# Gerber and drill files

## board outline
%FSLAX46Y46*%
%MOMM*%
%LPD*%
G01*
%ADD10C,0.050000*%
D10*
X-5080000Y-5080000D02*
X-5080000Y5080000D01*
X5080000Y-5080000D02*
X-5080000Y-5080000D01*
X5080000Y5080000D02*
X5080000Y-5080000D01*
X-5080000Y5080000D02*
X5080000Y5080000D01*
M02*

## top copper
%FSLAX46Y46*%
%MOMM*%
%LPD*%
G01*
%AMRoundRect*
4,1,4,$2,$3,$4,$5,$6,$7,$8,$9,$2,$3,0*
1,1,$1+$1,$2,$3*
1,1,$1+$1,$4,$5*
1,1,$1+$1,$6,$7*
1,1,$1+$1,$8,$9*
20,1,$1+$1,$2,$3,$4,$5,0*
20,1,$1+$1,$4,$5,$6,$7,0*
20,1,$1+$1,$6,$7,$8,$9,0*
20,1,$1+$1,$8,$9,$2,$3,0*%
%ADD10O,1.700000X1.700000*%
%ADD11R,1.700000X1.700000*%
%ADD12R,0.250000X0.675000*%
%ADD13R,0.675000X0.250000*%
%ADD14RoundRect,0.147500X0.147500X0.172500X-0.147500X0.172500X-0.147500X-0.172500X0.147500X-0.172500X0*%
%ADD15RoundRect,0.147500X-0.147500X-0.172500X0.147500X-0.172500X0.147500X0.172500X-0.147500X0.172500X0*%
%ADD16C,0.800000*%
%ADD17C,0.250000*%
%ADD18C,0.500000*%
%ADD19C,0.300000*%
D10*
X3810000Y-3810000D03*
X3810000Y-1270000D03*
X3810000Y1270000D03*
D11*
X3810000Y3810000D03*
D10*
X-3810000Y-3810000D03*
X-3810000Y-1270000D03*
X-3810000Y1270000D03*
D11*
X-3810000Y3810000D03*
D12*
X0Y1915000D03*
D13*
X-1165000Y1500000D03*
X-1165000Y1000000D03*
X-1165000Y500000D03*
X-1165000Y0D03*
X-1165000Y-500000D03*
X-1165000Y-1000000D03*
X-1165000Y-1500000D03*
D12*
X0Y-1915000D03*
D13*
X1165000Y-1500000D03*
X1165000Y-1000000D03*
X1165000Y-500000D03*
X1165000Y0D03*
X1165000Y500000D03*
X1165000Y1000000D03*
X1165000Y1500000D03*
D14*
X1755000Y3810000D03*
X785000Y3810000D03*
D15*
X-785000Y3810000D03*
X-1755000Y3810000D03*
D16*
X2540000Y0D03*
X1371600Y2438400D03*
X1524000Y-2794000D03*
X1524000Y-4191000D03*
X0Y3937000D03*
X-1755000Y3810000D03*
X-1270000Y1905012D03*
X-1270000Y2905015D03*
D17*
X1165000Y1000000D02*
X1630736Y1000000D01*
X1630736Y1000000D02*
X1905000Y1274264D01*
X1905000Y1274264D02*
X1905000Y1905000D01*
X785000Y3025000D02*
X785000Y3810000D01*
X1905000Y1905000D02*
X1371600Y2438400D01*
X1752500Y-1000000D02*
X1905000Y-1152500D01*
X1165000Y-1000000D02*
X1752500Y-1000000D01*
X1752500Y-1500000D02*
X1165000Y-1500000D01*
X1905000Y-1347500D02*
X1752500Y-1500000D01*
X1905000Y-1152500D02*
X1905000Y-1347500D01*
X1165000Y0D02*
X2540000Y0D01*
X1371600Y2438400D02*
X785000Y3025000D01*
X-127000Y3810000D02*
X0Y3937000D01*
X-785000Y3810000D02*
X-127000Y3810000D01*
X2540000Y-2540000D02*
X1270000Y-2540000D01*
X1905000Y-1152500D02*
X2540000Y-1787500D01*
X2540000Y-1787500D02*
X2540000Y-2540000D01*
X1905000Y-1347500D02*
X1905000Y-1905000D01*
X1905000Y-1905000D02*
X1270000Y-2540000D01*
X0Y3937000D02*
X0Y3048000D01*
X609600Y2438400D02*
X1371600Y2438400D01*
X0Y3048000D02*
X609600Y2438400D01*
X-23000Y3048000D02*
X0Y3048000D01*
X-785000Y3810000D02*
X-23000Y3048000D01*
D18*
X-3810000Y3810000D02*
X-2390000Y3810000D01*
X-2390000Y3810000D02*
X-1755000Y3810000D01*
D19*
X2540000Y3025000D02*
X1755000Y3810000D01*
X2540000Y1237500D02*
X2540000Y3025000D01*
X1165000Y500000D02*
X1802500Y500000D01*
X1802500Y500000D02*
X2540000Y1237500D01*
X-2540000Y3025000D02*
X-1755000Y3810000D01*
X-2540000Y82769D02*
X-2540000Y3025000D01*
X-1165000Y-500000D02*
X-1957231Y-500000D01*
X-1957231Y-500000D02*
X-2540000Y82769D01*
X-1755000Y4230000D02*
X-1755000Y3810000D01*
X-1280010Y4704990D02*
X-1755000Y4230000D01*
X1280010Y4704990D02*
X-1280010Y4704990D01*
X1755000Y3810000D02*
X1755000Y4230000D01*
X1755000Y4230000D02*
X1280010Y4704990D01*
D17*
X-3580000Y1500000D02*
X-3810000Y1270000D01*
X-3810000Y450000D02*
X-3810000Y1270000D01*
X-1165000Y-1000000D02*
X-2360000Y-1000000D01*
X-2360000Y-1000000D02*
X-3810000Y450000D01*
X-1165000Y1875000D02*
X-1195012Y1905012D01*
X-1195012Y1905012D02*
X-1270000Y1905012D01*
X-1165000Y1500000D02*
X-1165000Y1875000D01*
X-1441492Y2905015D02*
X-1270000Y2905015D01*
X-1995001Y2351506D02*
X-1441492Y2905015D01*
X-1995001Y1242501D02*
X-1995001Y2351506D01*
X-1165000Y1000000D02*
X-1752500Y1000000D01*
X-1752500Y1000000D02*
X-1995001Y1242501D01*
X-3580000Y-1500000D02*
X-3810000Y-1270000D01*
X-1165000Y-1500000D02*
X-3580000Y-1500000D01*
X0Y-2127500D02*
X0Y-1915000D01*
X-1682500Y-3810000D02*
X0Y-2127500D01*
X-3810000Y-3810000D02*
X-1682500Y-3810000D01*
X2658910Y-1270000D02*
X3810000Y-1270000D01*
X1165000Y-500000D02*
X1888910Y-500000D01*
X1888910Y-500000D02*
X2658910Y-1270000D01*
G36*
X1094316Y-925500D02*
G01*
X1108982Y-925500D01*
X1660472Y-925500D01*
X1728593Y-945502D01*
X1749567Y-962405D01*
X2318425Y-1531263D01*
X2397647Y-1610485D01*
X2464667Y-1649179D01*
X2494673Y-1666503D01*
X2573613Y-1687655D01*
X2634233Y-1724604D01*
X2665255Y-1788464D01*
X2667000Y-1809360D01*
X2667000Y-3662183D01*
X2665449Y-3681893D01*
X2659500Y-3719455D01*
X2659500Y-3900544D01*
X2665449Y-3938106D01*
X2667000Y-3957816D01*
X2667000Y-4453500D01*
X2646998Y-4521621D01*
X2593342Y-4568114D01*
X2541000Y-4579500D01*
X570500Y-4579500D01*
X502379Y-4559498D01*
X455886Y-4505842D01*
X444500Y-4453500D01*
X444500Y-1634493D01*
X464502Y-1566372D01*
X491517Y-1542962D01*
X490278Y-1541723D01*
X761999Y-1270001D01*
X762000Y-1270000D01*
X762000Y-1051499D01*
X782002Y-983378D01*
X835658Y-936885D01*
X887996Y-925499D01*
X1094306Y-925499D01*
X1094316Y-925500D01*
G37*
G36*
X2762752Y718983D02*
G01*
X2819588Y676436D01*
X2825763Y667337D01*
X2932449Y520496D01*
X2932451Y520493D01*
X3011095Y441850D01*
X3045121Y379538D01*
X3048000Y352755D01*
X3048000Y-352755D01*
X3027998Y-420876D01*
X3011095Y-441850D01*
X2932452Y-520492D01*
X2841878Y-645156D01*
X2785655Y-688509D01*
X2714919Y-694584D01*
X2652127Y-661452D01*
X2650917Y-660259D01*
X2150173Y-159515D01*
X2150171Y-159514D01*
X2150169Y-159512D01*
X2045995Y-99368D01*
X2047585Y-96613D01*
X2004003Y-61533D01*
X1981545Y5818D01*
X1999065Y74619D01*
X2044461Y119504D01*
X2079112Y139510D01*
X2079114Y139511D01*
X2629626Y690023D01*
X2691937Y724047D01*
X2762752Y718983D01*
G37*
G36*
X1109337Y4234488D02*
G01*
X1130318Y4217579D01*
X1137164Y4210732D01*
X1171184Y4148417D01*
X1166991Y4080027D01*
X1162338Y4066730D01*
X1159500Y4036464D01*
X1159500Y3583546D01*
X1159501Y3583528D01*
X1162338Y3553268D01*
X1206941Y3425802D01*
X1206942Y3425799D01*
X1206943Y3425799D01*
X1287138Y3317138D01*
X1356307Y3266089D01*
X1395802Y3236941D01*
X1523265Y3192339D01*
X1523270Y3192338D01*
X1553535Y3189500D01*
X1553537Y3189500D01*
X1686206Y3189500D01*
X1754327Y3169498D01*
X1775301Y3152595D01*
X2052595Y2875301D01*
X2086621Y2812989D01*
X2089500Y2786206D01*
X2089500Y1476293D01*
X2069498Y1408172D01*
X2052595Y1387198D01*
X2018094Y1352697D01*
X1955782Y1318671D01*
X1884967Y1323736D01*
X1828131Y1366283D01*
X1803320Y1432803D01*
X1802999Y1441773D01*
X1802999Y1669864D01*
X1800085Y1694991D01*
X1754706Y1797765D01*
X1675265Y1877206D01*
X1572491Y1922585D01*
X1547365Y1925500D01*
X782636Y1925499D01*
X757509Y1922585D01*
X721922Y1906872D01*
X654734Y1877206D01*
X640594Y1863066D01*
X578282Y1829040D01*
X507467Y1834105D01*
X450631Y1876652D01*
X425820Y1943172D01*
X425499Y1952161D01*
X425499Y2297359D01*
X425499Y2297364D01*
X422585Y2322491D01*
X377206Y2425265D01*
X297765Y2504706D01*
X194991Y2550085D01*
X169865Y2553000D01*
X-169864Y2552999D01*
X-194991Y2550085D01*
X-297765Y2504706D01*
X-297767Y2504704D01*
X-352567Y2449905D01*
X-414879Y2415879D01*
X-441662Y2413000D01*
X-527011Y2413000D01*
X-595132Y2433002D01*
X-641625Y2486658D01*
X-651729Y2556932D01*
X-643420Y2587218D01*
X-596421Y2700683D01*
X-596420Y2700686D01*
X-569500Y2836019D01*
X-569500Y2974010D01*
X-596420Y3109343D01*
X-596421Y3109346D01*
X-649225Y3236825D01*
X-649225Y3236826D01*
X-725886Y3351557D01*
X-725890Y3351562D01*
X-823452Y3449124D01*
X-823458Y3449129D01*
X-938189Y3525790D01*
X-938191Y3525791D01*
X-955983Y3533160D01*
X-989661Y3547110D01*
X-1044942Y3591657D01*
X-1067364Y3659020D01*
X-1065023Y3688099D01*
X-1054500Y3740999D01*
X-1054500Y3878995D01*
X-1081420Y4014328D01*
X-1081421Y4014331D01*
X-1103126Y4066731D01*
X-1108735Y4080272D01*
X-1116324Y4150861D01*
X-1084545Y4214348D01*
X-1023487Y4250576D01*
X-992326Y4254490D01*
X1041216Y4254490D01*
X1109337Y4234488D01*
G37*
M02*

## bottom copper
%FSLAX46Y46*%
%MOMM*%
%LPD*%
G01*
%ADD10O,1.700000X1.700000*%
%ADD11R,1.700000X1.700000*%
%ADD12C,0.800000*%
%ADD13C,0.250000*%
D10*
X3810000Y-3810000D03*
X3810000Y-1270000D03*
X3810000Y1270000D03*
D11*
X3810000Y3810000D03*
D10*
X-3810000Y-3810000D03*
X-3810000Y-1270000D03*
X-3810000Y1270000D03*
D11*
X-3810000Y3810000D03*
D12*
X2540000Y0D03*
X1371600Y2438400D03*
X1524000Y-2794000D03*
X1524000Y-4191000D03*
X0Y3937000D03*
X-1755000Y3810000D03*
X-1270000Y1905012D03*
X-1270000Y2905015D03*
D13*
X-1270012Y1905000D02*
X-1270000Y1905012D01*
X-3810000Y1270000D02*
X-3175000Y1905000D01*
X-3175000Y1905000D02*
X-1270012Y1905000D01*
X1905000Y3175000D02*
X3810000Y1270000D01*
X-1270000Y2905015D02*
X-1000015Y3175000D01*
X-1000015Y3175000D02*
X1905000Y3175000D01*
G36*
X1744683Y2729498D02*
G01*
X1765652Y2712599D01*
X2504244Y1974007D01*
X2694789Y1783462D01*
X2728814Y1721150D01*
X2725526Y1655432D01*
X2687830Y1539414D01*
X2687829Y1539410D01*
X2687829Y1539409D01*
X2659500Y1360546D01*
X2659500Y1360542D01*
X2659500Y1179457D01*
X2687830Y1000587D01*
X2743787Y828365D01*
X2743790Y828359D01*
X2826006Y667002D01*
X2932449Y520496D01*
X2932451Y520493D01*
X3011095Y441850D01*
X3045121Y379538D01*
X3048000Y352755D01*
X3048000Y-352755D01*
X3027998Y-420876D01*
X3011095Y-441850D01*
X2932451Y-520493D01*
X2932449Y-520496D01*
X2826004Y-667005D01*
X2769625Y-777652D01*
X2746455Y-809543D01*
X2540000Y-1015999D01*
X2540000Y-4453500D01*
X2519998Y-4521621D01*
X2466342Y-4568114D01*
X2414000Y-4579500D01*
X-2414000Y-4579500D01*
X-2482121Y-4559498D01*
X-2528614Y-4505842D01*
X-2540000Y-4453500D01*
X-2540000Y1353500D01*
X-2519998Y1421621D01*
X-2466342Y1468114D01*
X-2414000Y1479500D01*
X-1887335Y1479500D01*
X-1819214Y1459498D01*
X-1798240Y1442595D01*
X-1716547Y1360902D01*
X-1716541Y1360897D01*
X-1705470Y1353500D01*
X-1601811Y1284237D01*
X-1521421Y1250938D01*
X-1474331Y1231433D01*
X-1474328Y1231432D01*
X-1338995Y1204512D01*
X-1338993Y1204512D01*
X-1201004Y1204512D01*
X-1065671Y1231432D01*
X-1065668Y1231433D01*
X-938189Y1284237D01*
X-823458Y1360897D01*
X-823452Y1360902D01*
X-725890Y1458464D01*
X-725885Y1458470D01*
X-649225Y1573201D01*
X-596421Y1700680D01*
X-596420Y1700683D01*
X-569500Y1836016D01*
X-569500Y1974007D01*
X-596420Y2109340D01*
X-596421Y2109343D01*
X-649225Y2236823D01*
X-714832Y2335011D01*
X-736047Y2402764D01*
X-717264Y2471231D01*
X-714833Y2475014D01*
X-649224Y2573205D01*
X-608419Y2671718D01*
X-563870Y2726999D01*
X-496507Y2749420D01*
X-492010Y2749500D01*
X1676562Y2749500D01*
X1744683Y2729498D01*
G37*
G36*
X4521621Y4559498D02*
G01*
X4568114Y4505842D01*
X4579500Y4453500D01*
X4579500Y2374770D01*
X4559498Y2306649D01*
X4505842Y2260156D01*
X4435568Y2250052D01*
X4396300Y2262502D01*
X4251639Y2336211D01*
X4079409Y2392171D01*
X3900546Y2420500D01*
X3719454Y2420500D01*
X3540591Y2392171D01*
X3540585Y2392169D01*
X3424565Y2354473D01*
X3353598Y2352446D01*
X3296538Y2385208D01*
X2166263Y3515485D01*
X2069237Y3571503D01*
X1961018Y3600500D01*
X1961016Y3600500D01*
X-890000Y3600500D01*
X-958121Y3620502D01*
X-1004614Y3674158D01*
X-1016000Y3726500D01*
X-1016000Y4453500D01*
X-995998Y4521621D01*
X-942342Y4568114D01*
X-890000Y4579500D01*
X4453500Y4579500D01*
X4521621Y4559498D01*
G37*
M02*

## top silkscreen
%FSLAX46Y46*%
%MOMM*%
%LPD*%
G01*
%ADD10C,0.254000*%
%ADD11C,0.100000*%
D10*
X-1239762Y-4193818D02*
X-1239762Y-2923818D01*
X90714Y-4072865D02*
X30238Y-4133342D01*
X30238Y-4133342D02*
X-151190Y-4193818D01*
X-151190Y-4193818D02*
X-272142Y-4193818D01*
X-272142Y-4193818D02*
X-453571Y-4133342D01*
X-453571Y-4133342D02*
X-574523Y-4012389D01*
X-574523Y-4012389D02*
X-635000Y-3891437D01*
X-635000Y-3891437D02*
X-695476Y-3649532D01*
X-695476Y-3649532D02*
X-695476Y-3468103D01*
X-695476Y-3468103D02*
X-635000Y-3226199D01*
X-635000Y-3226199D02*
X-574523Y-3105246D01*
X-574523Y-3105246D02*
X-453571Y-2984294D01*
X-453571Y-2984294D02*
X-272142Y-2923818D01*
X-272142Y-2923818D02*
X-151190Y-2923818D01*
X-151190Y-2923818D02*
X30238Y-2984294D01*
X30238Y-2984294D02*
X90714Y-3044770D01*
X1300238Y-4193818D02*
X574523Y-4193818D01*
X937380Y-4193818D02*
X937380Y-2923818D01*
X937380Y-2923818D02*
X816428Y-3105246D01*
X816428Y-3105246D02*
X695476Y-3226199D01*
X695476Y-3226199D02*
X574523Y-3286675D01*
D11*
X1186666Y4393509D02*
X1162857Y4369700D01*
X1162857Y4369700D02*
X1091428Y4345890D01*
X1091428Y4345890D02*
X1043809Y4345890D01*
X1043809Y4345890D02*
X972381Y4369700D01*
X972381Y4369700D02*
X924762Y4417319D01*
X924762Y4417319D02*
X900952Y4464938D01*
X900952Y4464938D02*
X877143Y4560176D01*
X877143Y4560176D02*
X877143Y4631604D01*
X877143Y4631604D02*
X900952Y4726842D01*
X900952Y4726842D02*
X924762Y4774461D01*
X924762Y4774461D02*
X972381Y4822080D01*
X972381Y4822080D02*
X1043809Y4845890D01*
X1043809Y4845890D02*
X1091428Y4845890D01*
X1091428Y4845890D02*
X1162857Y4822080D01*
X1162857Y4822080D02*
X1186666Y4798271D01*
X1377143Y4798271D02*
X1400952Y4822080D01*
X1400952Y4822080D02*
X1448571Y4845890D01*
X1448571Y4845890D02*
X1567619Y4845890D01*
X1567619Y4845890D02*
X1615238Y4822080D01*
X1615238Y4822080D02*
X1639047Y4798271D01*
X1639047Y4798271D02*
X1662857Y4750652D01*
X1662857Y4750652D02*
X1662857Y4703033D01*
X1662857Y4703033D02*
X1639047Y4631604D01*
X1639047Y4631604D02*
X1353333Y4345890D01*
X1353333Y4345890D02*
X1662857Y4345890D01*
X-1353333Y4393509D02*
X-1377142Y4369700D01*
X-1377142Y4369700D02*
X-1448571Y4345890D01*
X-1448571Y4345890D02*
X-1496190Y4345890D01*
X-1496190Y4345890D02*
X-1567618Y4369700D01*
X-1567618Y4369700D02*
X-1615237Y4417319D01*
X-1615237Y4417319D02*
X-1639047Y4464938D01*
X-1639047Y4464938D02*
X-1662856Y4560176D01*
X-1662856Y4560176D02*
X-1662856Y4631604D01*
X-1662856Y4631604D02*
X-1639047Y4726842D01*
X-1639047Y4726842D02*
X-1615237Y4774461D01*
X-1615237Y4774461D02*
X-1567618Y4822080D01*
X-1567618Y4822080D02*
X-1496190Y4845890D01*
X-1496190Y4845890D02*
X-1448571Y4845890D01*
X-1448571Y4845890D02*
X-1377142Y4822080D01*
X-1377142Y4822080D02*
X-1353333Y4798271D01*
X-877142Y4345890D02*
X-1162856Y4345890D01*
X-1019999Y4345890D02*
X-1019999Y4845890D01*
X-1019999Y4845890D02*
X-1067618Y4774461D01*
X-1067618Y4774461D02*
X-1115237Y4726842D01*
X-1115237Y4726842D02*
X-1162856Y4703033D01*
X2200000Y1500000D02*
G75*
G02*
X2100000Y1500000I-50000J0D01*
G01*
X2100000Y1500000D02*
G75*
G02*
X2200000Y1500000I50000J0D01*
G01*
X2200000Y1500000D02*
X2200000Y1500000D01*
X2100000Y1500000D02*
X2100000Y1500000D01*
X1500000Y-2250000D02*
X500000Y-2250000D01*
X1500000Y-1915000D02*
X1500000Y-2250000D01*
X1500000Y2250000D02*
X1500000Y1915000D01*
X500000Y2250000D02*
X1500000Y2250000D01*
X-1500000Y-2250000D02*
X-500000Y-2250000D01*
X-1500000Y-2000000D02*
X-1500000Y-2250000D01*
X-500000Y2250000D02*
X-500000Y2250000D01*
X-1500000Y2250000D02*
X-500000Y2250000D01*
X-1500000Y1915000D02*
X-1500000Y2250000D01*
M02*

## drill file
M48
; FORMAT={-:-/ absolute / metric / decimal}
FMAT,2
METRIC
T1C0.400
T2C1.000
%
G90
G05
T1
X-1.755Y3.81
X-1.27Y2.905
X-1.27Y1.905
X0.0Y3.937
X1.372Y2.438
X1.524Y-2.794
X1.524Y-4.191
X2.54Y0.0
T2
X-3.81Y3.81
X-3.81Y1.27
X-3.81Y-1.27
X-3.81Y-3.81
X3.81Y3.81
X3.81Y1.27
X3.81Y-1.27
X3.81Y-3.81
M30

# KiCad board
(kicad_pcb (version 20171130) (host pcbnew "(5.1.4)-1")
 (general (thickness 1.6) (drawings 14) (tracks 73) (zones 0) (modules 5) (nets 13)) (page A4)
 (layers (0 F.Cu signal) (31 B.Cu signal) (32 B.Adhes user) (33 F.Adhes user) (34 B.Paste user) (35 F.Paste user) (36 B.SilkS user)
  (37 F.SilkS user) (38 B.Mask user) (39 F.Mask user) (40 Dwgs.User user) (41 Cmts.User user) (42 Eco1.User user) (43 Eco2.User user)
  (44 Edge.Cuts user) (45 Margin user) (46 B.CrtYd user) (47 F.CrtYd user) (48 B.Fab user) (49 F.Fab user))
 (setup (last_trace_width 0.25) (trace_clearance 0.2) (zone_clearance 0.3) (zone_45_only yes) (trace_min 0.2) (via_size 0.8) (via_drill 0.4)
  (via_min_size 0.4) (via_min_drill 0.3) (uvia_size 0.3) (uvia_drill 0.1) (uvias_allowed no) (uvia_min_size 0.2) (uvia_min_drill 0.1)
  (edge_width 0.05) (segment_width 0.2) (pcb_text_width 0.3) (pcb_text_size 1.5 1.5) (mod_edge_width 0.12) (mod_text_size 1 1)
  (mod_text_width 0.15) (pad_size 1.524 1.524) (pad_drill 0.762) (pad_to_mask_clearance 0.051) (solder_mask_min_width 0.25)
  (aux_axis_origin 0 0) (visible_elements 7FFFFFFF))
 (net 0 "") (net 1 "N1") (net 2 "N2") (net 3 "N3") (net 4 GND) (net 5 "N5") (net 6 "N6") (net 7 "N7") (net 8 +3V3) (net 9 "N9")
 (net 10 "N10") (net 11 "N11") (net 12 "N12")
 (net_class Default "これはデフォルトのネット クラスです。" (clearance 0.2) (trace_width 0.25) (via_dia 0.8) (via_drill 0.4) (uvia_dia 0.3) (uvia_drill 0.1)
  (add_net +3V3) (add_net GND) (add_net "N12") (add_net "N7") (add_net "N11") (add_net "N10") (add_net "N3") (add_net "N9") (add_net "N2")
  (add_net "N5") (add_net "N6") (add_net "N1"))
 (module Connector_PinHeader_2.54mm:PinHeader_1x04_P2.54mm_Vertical (layer B.Cu) (at 3.81 -3.81 180)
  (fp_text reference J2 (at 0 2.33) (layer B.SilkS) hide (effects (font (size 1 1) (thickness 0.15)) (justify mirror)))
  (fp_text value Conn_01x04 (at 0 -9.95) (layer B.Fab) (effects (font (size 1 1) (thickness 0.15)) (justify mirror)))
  (pad 4 thru_hole oval (at 0 -7.62 180) (size 1.7 1.7) (drill 1) (layers *.Cu *.Mask) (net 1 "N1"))
  (pad 3 thru_hole oval (at 0 -5.08 180) (size 1.7 1.7) (drill 1) (layers *.Cu *.Mask) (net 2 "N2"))
  (pad 2 thru_hole oval (at 0 -2.54 180) (size 1.7 1.7) (drill 1) (layers *.Cu *.Mask) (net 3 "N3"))
  (pad 1 thru_hole rect (at 0 0 180) (size 1.7 1.7) (drill 1) (layers *.Cu *.Mask) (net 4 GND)))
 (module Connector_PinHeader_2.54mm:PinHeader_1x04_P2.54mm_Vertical (layer B.Cu) (at -3.81 -3.81 180)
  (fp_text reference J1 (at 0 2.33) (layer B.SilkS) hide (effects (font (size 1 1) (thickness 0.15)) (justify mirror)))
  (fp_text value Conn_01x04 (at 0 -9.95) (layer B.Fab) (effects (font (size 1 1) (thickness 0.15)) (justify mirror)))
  (pad 4 thru_hole oval (at 0 -7.62 180) (size 1.7 1.7) (drill 1) (layers *.Cu *.Mask) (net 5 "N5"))
  (pad 3 thru_hole oval (at 0 -5.08 180) (size 1.7 1.7) (drill 1) (layers *.Cu *.Mask) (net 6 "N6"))
  (pad 2 thru_hole oval (at 0 -2.54 180) (size 1.7 1.7) (drill 1) (layers *.Cu *.Mask) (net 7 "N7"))
  (pad 1 thru_hole rect (at 0 0 180) (size 1.7 1.7) (drill 1) (layers *.Cu *.Mask) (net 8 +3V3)))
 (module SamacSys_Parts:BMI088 (layer F.Cu) (at 0 0 270)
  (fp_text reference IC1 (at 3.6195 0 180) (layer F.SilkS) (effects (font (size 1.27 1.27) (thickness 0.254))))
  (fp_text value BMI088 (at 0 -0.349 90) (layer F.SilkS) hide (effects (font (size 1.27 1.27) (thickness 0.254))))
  (fp_arc (start -1.5 -2.15) (end -1.5 -2.2) (angle 180) (layer F.SilkS) (width 0.1))
  (fp_arc (start -1.5 -2.15) (end -1.5 -2.1) (angle 180) (layer F.SilkS) (width 0.1))
  (fp_line (start -1.5 -2.2) (end -1.5 -2.2) (layer F.SilkS) (width 0.1))
  (fp_line (start -1.5 -2.1) (end -1.5 -2.1) (layer F.SilkS) (width 0.1))
  (fp_line (start 2.25 -1.5) (end 2.25 -0.5) (layer F.SilkS) (width 0.1))
  (fp_line (start 1.915 -1.5) (end 2.25 -1.5) (layer F.SilkS) (width 0.1))
  (fp_line (start -2.25 -1.5) (end -1.915 -1.5) (layer F.SilkS) (width 0.1))
  (fp_line (start -2.25 -0.5) (end -2.25 -1.5) (layer F.SilkS) (width 0.1))
  (fp_line (start 2.25 1.5) (end 2.25 0.5) (layer F.SilkS) (width 0.1))
  (fp_line (start 2 1.5) (end 2.25 1.5) (layer F.SilkS) (width 0.1))
  (fp_line (start -2.25 0.5) (end -2.25 0.5) (layer F.SilkS) (width 0.1))
  (fp_line (start -2.25 1.5) (end -2.25 0.5) (layer F.SilkS) (width 0.1))
  (fp_line (start -1.915 1.5) (end -2.25 1.5) (layer F.SilkS) (width 0.1))
  (pad 16 smd rect (at -1.915 0) (size 0.25 0.675) (layers F.Cu F.Paste F.Mask) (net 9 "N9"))
  (pad 15 smd rect (at -1.5 1.165 270) (size 0.25 0.675) (layers F.Cu F.Paste F.Mask) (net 7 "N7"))
  (pad 14 smd rect (at -1 1.165 270) (size 0.25 0.675) (layers F.Cu F.Paste F.Mask) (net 3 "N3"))
  (pad 13 smd rect (at -0.5 1.165 270) (size 0.25 0.675) (layers F.Cu F.Paste F.Mask) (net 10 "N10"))
  (pad 12 smd rect (at 0 1.165 270) (size 0.25 0.675) (layers F.Cu F.Paste F.Mask) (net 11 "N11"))
  (pad 11 smd rect (at 0.5 1.165 270) (size 0.25 0.675) (layers F.Cu F.Paste F.Mask) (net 8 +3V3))
  (pad 10 smd rect (at 1 1.165 270) (size 0.25 0.675) (layers F.Cu F.Paste F.Mask) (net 7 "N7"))
  (pad 9 smd rect (at 1.5 1.165 270) (size 0.25 0.675) (layers F.Cu F.Paste F.Mask) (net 6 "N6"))
  (pad 8 smd rect (at 1.915 0) (size 0.25 0.675) (layers F.Cu F.Paste F.Mask) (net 5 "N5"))
  (pad 7 smd rect (at 1.5 -1.165 270) (size 0.25 0.675) (layers F.Cu F.Paste F.Mask) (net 4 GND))
  (pad 6 smd rect (at 1 -1.165 270) (size 0.25 0.675) (layers F.Cu F.Paste F.Mask) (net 4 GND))
  (pad 5 smd rect (at 0.5 -1.165 270) (size 0.25 0.675) (layers F.Cu F.Paste F.Mask) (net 2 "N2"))
  (pad 4 smd rect (at 0 -1.165 270) (size 0.25 0.675) (layers F.Cu F.Paste F.Mask) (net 4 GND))
  (pad 3 smd rect (at -0.5 -1.165 270) (size 0.25 0.675) (layers F.Cu F.Paste F.Mask) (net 8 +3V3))
  (pad 2 smd rect (at -1 -1.165 270) (size 0.25 0.675) (layers F.Cu F.Paste F.Mask) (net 4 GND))
  (pad 1 smd rect (at -1.5 -1.165 270) (size 0.25 0.675) (layers F.Cu F.Paste F.Mask) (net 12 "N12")))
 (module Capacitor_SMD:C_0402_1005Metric (layer F.Cu) (at 1.27 -3.81 180)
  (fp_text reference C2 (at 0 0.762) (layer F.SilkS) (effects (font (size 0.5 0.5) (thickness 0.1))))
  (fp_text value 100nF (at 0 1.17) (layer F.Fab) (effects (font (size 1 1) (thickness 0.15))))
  (pad 1 smd roundrect (at -0.485 0 180) (size 0.59 0.64) (layers F.Cu F.Paste F.Mask) (roundrect_rratio 0.25) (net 8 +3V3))
  (pad 2 smd roundrect (at 0.485 0 180) (size 0.59 0.64) (layers F.Cu F.Paste F.Mask) (roundrect_rratio 0.25) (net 4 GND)))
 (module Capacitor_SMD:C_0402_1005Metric (layer F.Cu) (at -1.27 -3.81)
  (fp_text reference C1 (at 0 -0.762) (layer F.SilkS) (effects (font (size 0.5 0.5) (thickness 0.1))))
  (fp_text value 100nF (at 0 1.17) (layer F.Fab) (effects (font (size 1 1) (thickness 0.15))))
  (pad 2 smd roundrect (at 0.485 0) (size 0.59 0.64) (layers F.Cu F.Paste F.Mask) (roundrect_rratio 0.25) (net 4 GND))
  (pad 1 smd roundrect (at -0.485 0) (size 0.59 0.64) (layers F.Cu F.Paste F.Mask) (roundrect_rratio 0.25) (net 8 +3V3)))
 (gr_line (start -5.08 5.08) (end -5.08 -5.08) (layer Edge.Cuts) (width 0.05))
 (gr_line (start 5.08 5.08) (end -5.08 5.08) (layer Edge.Cuts) (width 0.05))
 (gr_line (start 5.08 -5.08) (end 5.08 5.08) (layer Edge.Cuts) (width 0.05))
 (gr_line (start -5.08 -5.08) (end 5.08 -5.08) (layer Edge.Cuts) (width 0.05))
 (segment (start 1.165 -1) (end 1.630736 -1) (width 0.25) (layer F.Cu) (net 4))
 (segment (start 1.630736 -1) (end 1.905 -1.274264) (width 0.25) (layer F.Cu) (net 4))
 (segment (start 1.905 -1.274264) (end 1.905 -1.905) (width 0.25) (layer F.Cu) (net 4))
 (segment (start 0.785 -3.025) (end 0.785 -3.81) (width 0.25) (layer F.Cu) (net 4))
 (segment (start 1.905 -1.905) (end 1.3716 -2.4384) (width 0.25) (layer F.Cu) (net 4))
 (segment (start 1.7525 1) (end 1.905 1.1525) (width 0.25) (layer F.Cu) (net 4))
 (segment (start 1.165 1) (end 1.7525 1) (width 0.25) (layer F.Cu) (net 4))
 (segment (start 1.7525 1.5) (end 1.165 1.5) (width 0.25) (layer F.Cu) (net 4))
 (segment (start 1.905 1.3475) (end 1.7525 1.5) (width 0.25) (layer F.Cu) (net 4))
 (segment (start 1.905 1.1525) (end 1.905 1.3475) (width 0.25) (layer F.Cu) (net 4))
 (via (at 2.54 0) (size 0.8) (drill 0.4) (layers F.Cu B.Cu) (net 4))
 (segment (start 1.165 0) (end 2.54 0) (width 0.25) (layer F.Cu) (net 4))
 (segment (start 1.3716 -2.4384) (end 0.785 -3.025) (width 0.25) (layer F.Cu) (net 4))
 (via (at 1.3716 -2.4384) (size 0.8) (drill 0.4) (layers F.Cu B.Cu) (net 4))
 (via (at 1.524 2.794) (size 0.8) (drill 0.4) (layers F.Cu B.Cu) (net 4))
 (via (at 1.524 4.191) (size 0.8) (drill 0.4) (layers F.Cu B.Cu) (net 4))
 (via (at 0 -3.937) (size 0.8) (drill 0.4) (layers F.Cu B.Cu) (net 4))
 (segment (start -0.127 -3.81) (end 0 -3.937) (width 0.25) (layer F.Cu) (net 4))
 (segment (start -0.785 -3.81) (end -0.127 -3.81) (width 0.25) (layer F.Cu) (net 4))
 (segment (start 2.54 2.54) (end 1.27 2.54) (width 0.25) (layer F.Cu) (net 4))
 (segment (start 1.905 1.1525) (end 2.54 1.7875) (width 0.25) (layer F.Cu) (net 4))
 (segment (start 2.54 1.7875) (end 2.54 2.54) (width 0.25) (layer F.Cu) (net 4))
 (segment (start 1.905 1.3475) (end 1.905 1.905) (width 0.25) (layer F.Cu) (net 4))
 (segment (start 1.905 1.905) (end 1.27 2.54) (width 0.25) (layer F.Cu) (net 4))
 (segment (start 0 -3.937) (end 0 -3.048) (width 0.25) (layer F.Cu) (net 4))
 (segment (start 0.6096 -2.4384) (end 1.3716 -2.4384) (width 0.25) (layer F.Cu) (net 4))
 (segment (start 0 -3.048) (end 0.6096 -2.4384) (width 0.25) (layer F.Cu) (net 4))
 (segment (start -0.023 -3.048) (end 0 -3.048) (width 0.25) (layer F.Cu) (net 4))
 (segment (start -0.785 -3.81) (end -0.023 -3.048) (width 0.25) (layer F.Cu) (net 4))
 (segment (start -3.81 -3.81) (end -2.39 -3.81) (width 0.5) (layer F.Cu) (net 8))
 (segment (start -2.39 -3.81) (end -1.755 -3.81) (width 0.5) (layer F.Cu) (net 8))
 (segment (start 2.54 -3.025) (end 1.755 -3.81) (width 0.3) (layer F.Cu) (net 8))
 (segment (start 2.54 -1.2375) (end 2.54 -3.025) (width 0.3) (layer F.Cu) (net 8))
 (segment (start 1.165 -0.5) (end 1.8025 -0.5) (width 0.3) (layer F.Cu) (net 8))
 (segment (start 1.8025 -0.5) (end 2.54 -1.2375) (width 0.3) (layer F.Cu) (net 8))
 (via (at -1.755 -3.81) (size 0.8) (drill 0.4) (layers F.Cu B.Cu) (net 8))
 (segment (start -2.54 -3.025) (end -1.755 -3.81) (width 0.3) (layer F.Cu) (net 8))
 (segment (start -2.54 -0.082769) (end -2.54 -3.025) (width 0.3) (layer F.Cu) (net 8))
 (segment (start -1.165 0.5) (end -1.957231 0.5) (width 0.3) (layer F.Cu) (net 8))
 (segment (start -1.957231 0.5) (end -2.54 -0.082769) (width 0.3) (layer F.Cu) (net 8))
 (segment (start -1.755 -4.23) (end -1.755 -3.81) (width 0.3) (layer F.Cu) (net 8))
 (segment (start -1.28001 -4.70499) (end -1.755 -4.23) (width 0.3) (layer F.Cu) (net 8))
 (segment (start 1.28001 -4.70499) (end -1.28001 -4.70499) (width 0.3) (layer F.Cu) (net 8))
 (segment (start 1.755 -3.81) (end 1.755 -4.23) (width 0.3) (layer F.Cu) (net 8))
 (segment (start 1.755 -4.23) (end 1.28001 -4.70499) (width 0.3) (layer F.Cu) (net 8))
 (segment (start -3.58 -1.5) (end -3.81 -1.27) (width 0.25) (layer F.Cu) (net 7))
 (segment (start -3.81 -0.45) (end -3.81 -1.27) (width 0.25) (layer F.Cu) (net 7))
 (segment (start -1.165 1) (end -2.36 1) (width 0.25) (layer F.Cu) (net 7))
 (segment (start -2.36 1) (end -3.81 -0.45) (width 0.25) (layer F.Cu) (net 7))
 (via (at -1.27 -1.905012) (size 0.8) (drill 0.4) (layers F.Cu B.Cu) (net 7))
 (segment (start -1.165 -1.875) (end -1.195012 -1.905012) (width 0.25) (layer F.Cu) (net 7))
 (segment (start -1.195012 -1.905012) (end -1.27 -1.905012) (width 0.25) (layer F.Cu) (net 7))
 (segment (start -1.165 -1.5) (end -1.165 -1.875) (width 0.25) (layer F.Cu) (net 7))
 (segment (start -1.270012 -1.905) (end -1.27 -1.905012) (width 0.25) (layer B.Cu) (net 7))
 (segment (start -3.81 -1.27) (end -3.175 -1.905) (width 0.25) (layer B.Cu) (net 7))
 (segment (start -3.175 -1.905) (end -1.270012 -1.905) (width 0.25) (layer B.Cu) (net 7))
 (via (at -1.27 -2.905015) (size 0.8) (drill 0.4) (layers F.Cu B.Cu) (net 3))
 (segment (start -1.441492 -2.905015) (end -1.27 -2.905015) (width 0.25) (layer F.Cu) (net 3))
 (segment (start -1.995001 -2.351506) (end -1.441492 -2.905015) (width 0.25) (layer F.Cu) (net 3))
 (segment (start -1.995001 -1.242501) (end -1.995001 -2.351506) (width 0.25) (layer F.Cu) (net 3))
 (segment (start -1.165 -1) (end -1.7525 -1) (width 0.25) (layer F.Cu) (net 3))
 (segment (start -1.7525 -1) (end -1.995001 -1.242501) (width 0.25) (layer F.Cu) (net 3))
 (segment (start 1.905 -3.175) (end 3.81 -1.27) (width 0.25) (layer B.Cu) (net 3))
 (segment (start -1.27 -2.905015) (end -1.000015 -3.175) (width 0.25) (layer B.Cu) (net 3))
 (segment (start -1.000015 -3.175) (end 1.905 -3.175) (width 0.25) (layer B.Cu) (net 3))
 (segment (start -3.58 1.5) (end -3.81 1.27) (width 0.25) (layer F.Cu) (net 6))
 (segment (start -1.165 1.5) (end -3.58 1.5) (width 0.25) (layer F.Cu) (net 6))
 (segment (start 0 2.1275) (end 0 1.915) (width 0.25) (layer F.Cu) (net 5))
 (segment (start -1.6825 3.81) (end 0 2.1275) (width 0.25) (layer F.Cu) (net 5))
 (segment (start -3.81 3.81) (end -1.6825 3.81) (width 0.25) (layer F.Cu) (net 5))
 (segment (start 2.65891 1.27) (end 3.81 1.27) (width 0.25) (layer F.Cu) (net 2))
 (segment (start 1.165 0.5) (end 1.88891 0.5) (width 0.25) (layer F.Cu) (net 2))
 (segment (start 1.88891 0.5) (end 2.65891 1.27) (width 0.25) (layer F.Cu) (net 2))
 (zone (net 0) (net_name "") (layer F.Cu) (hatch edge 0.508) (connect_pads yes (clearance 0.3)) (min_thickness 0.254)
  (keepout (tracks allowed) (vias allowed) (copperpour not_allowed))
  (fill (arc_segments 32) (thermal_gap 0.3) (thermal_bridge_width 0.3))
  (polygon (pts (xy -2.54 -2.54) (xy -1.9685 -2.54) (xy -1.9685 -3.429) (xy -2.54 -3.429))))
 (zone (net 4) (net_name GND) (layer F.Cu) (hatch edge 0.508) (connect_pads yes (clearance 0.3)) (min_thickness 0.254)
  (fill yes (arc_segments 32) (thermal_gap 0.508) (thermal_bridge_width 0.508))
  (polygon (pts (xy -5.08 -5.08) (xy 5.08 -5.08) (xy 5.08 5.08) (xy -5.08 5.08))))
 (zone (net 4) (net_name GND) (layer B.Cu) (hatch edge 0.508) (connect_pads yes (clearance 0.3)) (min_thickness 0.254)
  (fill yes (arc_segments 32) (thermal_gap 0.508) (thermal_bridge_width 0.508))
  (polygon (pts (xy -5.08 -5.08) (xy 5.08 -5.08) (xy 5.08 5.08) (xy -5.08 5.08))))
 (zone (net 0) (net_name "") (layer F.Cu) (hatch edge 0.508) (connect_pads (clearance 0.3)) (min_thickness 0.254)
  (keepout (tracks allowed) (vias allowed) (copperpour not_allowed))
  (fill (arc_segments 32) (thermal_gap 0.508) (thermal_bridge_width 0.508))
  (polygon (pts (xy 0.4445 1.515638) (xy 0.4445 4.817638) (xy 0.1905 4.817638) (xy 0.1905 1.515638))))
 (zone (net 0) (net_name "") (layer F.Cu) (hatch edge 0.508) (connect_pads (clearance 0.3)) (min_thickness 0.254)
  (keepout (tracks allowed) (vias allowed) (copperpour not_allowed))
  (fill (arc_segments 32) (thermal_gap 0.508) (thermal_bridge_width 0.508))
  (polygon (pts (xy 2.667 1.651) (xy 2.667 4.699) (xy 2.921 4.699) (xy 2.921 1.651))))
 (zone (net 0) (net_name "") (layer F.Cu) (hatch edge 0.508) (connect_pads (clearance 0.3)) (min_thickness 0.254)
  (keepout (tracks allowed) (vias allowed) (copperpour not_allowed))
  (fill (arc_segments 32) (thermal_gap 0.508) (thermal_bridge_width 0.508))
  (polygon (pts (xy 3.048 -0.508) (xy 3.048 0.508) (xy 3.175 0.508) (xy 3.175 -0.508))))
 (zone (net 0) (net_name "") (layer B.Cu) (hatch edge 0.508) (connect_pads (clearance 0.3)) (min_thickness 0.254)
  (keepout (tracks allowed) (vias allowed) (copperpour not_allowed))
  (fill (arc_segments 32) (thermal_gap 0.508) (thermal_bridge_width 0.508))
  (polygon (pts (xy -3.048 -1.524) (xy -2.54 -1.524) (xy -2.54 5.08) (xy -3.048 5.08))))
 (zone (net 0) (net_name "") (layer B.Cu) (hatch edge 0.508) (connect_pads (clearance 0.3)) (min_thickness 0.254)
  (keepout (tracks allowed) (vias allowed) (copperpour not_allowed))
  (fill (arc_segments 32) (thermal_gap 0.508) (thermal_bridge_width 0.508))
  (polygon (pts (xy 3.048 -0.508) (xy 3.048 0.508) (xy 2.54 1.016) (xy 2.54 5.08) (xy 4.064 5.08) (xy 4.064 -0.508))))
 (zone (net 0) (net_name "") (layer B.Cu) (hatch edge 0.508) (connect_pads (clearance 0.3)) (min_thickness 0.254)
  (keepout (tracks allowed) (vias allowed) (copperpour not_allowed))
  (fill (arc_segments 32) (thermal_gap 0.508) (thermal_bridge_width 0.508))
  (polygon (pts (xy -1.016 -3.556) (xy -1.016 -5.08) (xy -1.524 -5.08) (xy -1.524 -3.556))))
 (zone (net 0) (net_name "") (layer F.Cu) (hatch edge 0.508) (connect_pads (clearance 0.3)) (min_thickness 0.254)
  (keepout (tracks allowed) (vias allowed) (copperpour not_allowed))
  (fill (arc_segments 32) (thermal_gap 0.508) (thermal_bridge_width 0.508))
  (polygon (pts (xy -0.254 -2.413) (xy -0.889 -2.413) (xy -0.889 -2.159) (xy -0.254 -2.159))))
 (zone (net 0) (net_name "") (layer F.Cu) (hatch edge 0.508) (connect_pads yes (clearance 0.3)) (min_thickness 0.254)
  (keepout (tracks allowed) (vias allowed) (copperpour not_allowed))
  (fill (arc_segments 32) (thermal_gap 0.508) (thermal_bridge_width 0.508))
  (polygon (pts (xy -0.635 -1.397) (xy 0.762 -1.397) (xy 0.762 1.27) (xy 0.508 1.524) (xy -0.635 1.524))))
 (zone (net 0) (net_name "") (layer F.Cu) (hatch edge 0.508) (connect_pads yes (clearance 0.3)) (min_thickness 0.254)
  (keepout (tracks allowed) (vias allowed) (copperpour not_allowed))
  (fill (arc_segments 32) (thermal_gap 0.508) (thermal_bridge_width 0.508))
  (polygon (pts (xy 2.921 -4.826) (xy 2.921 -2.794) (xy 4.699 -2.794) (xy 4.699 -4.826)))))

